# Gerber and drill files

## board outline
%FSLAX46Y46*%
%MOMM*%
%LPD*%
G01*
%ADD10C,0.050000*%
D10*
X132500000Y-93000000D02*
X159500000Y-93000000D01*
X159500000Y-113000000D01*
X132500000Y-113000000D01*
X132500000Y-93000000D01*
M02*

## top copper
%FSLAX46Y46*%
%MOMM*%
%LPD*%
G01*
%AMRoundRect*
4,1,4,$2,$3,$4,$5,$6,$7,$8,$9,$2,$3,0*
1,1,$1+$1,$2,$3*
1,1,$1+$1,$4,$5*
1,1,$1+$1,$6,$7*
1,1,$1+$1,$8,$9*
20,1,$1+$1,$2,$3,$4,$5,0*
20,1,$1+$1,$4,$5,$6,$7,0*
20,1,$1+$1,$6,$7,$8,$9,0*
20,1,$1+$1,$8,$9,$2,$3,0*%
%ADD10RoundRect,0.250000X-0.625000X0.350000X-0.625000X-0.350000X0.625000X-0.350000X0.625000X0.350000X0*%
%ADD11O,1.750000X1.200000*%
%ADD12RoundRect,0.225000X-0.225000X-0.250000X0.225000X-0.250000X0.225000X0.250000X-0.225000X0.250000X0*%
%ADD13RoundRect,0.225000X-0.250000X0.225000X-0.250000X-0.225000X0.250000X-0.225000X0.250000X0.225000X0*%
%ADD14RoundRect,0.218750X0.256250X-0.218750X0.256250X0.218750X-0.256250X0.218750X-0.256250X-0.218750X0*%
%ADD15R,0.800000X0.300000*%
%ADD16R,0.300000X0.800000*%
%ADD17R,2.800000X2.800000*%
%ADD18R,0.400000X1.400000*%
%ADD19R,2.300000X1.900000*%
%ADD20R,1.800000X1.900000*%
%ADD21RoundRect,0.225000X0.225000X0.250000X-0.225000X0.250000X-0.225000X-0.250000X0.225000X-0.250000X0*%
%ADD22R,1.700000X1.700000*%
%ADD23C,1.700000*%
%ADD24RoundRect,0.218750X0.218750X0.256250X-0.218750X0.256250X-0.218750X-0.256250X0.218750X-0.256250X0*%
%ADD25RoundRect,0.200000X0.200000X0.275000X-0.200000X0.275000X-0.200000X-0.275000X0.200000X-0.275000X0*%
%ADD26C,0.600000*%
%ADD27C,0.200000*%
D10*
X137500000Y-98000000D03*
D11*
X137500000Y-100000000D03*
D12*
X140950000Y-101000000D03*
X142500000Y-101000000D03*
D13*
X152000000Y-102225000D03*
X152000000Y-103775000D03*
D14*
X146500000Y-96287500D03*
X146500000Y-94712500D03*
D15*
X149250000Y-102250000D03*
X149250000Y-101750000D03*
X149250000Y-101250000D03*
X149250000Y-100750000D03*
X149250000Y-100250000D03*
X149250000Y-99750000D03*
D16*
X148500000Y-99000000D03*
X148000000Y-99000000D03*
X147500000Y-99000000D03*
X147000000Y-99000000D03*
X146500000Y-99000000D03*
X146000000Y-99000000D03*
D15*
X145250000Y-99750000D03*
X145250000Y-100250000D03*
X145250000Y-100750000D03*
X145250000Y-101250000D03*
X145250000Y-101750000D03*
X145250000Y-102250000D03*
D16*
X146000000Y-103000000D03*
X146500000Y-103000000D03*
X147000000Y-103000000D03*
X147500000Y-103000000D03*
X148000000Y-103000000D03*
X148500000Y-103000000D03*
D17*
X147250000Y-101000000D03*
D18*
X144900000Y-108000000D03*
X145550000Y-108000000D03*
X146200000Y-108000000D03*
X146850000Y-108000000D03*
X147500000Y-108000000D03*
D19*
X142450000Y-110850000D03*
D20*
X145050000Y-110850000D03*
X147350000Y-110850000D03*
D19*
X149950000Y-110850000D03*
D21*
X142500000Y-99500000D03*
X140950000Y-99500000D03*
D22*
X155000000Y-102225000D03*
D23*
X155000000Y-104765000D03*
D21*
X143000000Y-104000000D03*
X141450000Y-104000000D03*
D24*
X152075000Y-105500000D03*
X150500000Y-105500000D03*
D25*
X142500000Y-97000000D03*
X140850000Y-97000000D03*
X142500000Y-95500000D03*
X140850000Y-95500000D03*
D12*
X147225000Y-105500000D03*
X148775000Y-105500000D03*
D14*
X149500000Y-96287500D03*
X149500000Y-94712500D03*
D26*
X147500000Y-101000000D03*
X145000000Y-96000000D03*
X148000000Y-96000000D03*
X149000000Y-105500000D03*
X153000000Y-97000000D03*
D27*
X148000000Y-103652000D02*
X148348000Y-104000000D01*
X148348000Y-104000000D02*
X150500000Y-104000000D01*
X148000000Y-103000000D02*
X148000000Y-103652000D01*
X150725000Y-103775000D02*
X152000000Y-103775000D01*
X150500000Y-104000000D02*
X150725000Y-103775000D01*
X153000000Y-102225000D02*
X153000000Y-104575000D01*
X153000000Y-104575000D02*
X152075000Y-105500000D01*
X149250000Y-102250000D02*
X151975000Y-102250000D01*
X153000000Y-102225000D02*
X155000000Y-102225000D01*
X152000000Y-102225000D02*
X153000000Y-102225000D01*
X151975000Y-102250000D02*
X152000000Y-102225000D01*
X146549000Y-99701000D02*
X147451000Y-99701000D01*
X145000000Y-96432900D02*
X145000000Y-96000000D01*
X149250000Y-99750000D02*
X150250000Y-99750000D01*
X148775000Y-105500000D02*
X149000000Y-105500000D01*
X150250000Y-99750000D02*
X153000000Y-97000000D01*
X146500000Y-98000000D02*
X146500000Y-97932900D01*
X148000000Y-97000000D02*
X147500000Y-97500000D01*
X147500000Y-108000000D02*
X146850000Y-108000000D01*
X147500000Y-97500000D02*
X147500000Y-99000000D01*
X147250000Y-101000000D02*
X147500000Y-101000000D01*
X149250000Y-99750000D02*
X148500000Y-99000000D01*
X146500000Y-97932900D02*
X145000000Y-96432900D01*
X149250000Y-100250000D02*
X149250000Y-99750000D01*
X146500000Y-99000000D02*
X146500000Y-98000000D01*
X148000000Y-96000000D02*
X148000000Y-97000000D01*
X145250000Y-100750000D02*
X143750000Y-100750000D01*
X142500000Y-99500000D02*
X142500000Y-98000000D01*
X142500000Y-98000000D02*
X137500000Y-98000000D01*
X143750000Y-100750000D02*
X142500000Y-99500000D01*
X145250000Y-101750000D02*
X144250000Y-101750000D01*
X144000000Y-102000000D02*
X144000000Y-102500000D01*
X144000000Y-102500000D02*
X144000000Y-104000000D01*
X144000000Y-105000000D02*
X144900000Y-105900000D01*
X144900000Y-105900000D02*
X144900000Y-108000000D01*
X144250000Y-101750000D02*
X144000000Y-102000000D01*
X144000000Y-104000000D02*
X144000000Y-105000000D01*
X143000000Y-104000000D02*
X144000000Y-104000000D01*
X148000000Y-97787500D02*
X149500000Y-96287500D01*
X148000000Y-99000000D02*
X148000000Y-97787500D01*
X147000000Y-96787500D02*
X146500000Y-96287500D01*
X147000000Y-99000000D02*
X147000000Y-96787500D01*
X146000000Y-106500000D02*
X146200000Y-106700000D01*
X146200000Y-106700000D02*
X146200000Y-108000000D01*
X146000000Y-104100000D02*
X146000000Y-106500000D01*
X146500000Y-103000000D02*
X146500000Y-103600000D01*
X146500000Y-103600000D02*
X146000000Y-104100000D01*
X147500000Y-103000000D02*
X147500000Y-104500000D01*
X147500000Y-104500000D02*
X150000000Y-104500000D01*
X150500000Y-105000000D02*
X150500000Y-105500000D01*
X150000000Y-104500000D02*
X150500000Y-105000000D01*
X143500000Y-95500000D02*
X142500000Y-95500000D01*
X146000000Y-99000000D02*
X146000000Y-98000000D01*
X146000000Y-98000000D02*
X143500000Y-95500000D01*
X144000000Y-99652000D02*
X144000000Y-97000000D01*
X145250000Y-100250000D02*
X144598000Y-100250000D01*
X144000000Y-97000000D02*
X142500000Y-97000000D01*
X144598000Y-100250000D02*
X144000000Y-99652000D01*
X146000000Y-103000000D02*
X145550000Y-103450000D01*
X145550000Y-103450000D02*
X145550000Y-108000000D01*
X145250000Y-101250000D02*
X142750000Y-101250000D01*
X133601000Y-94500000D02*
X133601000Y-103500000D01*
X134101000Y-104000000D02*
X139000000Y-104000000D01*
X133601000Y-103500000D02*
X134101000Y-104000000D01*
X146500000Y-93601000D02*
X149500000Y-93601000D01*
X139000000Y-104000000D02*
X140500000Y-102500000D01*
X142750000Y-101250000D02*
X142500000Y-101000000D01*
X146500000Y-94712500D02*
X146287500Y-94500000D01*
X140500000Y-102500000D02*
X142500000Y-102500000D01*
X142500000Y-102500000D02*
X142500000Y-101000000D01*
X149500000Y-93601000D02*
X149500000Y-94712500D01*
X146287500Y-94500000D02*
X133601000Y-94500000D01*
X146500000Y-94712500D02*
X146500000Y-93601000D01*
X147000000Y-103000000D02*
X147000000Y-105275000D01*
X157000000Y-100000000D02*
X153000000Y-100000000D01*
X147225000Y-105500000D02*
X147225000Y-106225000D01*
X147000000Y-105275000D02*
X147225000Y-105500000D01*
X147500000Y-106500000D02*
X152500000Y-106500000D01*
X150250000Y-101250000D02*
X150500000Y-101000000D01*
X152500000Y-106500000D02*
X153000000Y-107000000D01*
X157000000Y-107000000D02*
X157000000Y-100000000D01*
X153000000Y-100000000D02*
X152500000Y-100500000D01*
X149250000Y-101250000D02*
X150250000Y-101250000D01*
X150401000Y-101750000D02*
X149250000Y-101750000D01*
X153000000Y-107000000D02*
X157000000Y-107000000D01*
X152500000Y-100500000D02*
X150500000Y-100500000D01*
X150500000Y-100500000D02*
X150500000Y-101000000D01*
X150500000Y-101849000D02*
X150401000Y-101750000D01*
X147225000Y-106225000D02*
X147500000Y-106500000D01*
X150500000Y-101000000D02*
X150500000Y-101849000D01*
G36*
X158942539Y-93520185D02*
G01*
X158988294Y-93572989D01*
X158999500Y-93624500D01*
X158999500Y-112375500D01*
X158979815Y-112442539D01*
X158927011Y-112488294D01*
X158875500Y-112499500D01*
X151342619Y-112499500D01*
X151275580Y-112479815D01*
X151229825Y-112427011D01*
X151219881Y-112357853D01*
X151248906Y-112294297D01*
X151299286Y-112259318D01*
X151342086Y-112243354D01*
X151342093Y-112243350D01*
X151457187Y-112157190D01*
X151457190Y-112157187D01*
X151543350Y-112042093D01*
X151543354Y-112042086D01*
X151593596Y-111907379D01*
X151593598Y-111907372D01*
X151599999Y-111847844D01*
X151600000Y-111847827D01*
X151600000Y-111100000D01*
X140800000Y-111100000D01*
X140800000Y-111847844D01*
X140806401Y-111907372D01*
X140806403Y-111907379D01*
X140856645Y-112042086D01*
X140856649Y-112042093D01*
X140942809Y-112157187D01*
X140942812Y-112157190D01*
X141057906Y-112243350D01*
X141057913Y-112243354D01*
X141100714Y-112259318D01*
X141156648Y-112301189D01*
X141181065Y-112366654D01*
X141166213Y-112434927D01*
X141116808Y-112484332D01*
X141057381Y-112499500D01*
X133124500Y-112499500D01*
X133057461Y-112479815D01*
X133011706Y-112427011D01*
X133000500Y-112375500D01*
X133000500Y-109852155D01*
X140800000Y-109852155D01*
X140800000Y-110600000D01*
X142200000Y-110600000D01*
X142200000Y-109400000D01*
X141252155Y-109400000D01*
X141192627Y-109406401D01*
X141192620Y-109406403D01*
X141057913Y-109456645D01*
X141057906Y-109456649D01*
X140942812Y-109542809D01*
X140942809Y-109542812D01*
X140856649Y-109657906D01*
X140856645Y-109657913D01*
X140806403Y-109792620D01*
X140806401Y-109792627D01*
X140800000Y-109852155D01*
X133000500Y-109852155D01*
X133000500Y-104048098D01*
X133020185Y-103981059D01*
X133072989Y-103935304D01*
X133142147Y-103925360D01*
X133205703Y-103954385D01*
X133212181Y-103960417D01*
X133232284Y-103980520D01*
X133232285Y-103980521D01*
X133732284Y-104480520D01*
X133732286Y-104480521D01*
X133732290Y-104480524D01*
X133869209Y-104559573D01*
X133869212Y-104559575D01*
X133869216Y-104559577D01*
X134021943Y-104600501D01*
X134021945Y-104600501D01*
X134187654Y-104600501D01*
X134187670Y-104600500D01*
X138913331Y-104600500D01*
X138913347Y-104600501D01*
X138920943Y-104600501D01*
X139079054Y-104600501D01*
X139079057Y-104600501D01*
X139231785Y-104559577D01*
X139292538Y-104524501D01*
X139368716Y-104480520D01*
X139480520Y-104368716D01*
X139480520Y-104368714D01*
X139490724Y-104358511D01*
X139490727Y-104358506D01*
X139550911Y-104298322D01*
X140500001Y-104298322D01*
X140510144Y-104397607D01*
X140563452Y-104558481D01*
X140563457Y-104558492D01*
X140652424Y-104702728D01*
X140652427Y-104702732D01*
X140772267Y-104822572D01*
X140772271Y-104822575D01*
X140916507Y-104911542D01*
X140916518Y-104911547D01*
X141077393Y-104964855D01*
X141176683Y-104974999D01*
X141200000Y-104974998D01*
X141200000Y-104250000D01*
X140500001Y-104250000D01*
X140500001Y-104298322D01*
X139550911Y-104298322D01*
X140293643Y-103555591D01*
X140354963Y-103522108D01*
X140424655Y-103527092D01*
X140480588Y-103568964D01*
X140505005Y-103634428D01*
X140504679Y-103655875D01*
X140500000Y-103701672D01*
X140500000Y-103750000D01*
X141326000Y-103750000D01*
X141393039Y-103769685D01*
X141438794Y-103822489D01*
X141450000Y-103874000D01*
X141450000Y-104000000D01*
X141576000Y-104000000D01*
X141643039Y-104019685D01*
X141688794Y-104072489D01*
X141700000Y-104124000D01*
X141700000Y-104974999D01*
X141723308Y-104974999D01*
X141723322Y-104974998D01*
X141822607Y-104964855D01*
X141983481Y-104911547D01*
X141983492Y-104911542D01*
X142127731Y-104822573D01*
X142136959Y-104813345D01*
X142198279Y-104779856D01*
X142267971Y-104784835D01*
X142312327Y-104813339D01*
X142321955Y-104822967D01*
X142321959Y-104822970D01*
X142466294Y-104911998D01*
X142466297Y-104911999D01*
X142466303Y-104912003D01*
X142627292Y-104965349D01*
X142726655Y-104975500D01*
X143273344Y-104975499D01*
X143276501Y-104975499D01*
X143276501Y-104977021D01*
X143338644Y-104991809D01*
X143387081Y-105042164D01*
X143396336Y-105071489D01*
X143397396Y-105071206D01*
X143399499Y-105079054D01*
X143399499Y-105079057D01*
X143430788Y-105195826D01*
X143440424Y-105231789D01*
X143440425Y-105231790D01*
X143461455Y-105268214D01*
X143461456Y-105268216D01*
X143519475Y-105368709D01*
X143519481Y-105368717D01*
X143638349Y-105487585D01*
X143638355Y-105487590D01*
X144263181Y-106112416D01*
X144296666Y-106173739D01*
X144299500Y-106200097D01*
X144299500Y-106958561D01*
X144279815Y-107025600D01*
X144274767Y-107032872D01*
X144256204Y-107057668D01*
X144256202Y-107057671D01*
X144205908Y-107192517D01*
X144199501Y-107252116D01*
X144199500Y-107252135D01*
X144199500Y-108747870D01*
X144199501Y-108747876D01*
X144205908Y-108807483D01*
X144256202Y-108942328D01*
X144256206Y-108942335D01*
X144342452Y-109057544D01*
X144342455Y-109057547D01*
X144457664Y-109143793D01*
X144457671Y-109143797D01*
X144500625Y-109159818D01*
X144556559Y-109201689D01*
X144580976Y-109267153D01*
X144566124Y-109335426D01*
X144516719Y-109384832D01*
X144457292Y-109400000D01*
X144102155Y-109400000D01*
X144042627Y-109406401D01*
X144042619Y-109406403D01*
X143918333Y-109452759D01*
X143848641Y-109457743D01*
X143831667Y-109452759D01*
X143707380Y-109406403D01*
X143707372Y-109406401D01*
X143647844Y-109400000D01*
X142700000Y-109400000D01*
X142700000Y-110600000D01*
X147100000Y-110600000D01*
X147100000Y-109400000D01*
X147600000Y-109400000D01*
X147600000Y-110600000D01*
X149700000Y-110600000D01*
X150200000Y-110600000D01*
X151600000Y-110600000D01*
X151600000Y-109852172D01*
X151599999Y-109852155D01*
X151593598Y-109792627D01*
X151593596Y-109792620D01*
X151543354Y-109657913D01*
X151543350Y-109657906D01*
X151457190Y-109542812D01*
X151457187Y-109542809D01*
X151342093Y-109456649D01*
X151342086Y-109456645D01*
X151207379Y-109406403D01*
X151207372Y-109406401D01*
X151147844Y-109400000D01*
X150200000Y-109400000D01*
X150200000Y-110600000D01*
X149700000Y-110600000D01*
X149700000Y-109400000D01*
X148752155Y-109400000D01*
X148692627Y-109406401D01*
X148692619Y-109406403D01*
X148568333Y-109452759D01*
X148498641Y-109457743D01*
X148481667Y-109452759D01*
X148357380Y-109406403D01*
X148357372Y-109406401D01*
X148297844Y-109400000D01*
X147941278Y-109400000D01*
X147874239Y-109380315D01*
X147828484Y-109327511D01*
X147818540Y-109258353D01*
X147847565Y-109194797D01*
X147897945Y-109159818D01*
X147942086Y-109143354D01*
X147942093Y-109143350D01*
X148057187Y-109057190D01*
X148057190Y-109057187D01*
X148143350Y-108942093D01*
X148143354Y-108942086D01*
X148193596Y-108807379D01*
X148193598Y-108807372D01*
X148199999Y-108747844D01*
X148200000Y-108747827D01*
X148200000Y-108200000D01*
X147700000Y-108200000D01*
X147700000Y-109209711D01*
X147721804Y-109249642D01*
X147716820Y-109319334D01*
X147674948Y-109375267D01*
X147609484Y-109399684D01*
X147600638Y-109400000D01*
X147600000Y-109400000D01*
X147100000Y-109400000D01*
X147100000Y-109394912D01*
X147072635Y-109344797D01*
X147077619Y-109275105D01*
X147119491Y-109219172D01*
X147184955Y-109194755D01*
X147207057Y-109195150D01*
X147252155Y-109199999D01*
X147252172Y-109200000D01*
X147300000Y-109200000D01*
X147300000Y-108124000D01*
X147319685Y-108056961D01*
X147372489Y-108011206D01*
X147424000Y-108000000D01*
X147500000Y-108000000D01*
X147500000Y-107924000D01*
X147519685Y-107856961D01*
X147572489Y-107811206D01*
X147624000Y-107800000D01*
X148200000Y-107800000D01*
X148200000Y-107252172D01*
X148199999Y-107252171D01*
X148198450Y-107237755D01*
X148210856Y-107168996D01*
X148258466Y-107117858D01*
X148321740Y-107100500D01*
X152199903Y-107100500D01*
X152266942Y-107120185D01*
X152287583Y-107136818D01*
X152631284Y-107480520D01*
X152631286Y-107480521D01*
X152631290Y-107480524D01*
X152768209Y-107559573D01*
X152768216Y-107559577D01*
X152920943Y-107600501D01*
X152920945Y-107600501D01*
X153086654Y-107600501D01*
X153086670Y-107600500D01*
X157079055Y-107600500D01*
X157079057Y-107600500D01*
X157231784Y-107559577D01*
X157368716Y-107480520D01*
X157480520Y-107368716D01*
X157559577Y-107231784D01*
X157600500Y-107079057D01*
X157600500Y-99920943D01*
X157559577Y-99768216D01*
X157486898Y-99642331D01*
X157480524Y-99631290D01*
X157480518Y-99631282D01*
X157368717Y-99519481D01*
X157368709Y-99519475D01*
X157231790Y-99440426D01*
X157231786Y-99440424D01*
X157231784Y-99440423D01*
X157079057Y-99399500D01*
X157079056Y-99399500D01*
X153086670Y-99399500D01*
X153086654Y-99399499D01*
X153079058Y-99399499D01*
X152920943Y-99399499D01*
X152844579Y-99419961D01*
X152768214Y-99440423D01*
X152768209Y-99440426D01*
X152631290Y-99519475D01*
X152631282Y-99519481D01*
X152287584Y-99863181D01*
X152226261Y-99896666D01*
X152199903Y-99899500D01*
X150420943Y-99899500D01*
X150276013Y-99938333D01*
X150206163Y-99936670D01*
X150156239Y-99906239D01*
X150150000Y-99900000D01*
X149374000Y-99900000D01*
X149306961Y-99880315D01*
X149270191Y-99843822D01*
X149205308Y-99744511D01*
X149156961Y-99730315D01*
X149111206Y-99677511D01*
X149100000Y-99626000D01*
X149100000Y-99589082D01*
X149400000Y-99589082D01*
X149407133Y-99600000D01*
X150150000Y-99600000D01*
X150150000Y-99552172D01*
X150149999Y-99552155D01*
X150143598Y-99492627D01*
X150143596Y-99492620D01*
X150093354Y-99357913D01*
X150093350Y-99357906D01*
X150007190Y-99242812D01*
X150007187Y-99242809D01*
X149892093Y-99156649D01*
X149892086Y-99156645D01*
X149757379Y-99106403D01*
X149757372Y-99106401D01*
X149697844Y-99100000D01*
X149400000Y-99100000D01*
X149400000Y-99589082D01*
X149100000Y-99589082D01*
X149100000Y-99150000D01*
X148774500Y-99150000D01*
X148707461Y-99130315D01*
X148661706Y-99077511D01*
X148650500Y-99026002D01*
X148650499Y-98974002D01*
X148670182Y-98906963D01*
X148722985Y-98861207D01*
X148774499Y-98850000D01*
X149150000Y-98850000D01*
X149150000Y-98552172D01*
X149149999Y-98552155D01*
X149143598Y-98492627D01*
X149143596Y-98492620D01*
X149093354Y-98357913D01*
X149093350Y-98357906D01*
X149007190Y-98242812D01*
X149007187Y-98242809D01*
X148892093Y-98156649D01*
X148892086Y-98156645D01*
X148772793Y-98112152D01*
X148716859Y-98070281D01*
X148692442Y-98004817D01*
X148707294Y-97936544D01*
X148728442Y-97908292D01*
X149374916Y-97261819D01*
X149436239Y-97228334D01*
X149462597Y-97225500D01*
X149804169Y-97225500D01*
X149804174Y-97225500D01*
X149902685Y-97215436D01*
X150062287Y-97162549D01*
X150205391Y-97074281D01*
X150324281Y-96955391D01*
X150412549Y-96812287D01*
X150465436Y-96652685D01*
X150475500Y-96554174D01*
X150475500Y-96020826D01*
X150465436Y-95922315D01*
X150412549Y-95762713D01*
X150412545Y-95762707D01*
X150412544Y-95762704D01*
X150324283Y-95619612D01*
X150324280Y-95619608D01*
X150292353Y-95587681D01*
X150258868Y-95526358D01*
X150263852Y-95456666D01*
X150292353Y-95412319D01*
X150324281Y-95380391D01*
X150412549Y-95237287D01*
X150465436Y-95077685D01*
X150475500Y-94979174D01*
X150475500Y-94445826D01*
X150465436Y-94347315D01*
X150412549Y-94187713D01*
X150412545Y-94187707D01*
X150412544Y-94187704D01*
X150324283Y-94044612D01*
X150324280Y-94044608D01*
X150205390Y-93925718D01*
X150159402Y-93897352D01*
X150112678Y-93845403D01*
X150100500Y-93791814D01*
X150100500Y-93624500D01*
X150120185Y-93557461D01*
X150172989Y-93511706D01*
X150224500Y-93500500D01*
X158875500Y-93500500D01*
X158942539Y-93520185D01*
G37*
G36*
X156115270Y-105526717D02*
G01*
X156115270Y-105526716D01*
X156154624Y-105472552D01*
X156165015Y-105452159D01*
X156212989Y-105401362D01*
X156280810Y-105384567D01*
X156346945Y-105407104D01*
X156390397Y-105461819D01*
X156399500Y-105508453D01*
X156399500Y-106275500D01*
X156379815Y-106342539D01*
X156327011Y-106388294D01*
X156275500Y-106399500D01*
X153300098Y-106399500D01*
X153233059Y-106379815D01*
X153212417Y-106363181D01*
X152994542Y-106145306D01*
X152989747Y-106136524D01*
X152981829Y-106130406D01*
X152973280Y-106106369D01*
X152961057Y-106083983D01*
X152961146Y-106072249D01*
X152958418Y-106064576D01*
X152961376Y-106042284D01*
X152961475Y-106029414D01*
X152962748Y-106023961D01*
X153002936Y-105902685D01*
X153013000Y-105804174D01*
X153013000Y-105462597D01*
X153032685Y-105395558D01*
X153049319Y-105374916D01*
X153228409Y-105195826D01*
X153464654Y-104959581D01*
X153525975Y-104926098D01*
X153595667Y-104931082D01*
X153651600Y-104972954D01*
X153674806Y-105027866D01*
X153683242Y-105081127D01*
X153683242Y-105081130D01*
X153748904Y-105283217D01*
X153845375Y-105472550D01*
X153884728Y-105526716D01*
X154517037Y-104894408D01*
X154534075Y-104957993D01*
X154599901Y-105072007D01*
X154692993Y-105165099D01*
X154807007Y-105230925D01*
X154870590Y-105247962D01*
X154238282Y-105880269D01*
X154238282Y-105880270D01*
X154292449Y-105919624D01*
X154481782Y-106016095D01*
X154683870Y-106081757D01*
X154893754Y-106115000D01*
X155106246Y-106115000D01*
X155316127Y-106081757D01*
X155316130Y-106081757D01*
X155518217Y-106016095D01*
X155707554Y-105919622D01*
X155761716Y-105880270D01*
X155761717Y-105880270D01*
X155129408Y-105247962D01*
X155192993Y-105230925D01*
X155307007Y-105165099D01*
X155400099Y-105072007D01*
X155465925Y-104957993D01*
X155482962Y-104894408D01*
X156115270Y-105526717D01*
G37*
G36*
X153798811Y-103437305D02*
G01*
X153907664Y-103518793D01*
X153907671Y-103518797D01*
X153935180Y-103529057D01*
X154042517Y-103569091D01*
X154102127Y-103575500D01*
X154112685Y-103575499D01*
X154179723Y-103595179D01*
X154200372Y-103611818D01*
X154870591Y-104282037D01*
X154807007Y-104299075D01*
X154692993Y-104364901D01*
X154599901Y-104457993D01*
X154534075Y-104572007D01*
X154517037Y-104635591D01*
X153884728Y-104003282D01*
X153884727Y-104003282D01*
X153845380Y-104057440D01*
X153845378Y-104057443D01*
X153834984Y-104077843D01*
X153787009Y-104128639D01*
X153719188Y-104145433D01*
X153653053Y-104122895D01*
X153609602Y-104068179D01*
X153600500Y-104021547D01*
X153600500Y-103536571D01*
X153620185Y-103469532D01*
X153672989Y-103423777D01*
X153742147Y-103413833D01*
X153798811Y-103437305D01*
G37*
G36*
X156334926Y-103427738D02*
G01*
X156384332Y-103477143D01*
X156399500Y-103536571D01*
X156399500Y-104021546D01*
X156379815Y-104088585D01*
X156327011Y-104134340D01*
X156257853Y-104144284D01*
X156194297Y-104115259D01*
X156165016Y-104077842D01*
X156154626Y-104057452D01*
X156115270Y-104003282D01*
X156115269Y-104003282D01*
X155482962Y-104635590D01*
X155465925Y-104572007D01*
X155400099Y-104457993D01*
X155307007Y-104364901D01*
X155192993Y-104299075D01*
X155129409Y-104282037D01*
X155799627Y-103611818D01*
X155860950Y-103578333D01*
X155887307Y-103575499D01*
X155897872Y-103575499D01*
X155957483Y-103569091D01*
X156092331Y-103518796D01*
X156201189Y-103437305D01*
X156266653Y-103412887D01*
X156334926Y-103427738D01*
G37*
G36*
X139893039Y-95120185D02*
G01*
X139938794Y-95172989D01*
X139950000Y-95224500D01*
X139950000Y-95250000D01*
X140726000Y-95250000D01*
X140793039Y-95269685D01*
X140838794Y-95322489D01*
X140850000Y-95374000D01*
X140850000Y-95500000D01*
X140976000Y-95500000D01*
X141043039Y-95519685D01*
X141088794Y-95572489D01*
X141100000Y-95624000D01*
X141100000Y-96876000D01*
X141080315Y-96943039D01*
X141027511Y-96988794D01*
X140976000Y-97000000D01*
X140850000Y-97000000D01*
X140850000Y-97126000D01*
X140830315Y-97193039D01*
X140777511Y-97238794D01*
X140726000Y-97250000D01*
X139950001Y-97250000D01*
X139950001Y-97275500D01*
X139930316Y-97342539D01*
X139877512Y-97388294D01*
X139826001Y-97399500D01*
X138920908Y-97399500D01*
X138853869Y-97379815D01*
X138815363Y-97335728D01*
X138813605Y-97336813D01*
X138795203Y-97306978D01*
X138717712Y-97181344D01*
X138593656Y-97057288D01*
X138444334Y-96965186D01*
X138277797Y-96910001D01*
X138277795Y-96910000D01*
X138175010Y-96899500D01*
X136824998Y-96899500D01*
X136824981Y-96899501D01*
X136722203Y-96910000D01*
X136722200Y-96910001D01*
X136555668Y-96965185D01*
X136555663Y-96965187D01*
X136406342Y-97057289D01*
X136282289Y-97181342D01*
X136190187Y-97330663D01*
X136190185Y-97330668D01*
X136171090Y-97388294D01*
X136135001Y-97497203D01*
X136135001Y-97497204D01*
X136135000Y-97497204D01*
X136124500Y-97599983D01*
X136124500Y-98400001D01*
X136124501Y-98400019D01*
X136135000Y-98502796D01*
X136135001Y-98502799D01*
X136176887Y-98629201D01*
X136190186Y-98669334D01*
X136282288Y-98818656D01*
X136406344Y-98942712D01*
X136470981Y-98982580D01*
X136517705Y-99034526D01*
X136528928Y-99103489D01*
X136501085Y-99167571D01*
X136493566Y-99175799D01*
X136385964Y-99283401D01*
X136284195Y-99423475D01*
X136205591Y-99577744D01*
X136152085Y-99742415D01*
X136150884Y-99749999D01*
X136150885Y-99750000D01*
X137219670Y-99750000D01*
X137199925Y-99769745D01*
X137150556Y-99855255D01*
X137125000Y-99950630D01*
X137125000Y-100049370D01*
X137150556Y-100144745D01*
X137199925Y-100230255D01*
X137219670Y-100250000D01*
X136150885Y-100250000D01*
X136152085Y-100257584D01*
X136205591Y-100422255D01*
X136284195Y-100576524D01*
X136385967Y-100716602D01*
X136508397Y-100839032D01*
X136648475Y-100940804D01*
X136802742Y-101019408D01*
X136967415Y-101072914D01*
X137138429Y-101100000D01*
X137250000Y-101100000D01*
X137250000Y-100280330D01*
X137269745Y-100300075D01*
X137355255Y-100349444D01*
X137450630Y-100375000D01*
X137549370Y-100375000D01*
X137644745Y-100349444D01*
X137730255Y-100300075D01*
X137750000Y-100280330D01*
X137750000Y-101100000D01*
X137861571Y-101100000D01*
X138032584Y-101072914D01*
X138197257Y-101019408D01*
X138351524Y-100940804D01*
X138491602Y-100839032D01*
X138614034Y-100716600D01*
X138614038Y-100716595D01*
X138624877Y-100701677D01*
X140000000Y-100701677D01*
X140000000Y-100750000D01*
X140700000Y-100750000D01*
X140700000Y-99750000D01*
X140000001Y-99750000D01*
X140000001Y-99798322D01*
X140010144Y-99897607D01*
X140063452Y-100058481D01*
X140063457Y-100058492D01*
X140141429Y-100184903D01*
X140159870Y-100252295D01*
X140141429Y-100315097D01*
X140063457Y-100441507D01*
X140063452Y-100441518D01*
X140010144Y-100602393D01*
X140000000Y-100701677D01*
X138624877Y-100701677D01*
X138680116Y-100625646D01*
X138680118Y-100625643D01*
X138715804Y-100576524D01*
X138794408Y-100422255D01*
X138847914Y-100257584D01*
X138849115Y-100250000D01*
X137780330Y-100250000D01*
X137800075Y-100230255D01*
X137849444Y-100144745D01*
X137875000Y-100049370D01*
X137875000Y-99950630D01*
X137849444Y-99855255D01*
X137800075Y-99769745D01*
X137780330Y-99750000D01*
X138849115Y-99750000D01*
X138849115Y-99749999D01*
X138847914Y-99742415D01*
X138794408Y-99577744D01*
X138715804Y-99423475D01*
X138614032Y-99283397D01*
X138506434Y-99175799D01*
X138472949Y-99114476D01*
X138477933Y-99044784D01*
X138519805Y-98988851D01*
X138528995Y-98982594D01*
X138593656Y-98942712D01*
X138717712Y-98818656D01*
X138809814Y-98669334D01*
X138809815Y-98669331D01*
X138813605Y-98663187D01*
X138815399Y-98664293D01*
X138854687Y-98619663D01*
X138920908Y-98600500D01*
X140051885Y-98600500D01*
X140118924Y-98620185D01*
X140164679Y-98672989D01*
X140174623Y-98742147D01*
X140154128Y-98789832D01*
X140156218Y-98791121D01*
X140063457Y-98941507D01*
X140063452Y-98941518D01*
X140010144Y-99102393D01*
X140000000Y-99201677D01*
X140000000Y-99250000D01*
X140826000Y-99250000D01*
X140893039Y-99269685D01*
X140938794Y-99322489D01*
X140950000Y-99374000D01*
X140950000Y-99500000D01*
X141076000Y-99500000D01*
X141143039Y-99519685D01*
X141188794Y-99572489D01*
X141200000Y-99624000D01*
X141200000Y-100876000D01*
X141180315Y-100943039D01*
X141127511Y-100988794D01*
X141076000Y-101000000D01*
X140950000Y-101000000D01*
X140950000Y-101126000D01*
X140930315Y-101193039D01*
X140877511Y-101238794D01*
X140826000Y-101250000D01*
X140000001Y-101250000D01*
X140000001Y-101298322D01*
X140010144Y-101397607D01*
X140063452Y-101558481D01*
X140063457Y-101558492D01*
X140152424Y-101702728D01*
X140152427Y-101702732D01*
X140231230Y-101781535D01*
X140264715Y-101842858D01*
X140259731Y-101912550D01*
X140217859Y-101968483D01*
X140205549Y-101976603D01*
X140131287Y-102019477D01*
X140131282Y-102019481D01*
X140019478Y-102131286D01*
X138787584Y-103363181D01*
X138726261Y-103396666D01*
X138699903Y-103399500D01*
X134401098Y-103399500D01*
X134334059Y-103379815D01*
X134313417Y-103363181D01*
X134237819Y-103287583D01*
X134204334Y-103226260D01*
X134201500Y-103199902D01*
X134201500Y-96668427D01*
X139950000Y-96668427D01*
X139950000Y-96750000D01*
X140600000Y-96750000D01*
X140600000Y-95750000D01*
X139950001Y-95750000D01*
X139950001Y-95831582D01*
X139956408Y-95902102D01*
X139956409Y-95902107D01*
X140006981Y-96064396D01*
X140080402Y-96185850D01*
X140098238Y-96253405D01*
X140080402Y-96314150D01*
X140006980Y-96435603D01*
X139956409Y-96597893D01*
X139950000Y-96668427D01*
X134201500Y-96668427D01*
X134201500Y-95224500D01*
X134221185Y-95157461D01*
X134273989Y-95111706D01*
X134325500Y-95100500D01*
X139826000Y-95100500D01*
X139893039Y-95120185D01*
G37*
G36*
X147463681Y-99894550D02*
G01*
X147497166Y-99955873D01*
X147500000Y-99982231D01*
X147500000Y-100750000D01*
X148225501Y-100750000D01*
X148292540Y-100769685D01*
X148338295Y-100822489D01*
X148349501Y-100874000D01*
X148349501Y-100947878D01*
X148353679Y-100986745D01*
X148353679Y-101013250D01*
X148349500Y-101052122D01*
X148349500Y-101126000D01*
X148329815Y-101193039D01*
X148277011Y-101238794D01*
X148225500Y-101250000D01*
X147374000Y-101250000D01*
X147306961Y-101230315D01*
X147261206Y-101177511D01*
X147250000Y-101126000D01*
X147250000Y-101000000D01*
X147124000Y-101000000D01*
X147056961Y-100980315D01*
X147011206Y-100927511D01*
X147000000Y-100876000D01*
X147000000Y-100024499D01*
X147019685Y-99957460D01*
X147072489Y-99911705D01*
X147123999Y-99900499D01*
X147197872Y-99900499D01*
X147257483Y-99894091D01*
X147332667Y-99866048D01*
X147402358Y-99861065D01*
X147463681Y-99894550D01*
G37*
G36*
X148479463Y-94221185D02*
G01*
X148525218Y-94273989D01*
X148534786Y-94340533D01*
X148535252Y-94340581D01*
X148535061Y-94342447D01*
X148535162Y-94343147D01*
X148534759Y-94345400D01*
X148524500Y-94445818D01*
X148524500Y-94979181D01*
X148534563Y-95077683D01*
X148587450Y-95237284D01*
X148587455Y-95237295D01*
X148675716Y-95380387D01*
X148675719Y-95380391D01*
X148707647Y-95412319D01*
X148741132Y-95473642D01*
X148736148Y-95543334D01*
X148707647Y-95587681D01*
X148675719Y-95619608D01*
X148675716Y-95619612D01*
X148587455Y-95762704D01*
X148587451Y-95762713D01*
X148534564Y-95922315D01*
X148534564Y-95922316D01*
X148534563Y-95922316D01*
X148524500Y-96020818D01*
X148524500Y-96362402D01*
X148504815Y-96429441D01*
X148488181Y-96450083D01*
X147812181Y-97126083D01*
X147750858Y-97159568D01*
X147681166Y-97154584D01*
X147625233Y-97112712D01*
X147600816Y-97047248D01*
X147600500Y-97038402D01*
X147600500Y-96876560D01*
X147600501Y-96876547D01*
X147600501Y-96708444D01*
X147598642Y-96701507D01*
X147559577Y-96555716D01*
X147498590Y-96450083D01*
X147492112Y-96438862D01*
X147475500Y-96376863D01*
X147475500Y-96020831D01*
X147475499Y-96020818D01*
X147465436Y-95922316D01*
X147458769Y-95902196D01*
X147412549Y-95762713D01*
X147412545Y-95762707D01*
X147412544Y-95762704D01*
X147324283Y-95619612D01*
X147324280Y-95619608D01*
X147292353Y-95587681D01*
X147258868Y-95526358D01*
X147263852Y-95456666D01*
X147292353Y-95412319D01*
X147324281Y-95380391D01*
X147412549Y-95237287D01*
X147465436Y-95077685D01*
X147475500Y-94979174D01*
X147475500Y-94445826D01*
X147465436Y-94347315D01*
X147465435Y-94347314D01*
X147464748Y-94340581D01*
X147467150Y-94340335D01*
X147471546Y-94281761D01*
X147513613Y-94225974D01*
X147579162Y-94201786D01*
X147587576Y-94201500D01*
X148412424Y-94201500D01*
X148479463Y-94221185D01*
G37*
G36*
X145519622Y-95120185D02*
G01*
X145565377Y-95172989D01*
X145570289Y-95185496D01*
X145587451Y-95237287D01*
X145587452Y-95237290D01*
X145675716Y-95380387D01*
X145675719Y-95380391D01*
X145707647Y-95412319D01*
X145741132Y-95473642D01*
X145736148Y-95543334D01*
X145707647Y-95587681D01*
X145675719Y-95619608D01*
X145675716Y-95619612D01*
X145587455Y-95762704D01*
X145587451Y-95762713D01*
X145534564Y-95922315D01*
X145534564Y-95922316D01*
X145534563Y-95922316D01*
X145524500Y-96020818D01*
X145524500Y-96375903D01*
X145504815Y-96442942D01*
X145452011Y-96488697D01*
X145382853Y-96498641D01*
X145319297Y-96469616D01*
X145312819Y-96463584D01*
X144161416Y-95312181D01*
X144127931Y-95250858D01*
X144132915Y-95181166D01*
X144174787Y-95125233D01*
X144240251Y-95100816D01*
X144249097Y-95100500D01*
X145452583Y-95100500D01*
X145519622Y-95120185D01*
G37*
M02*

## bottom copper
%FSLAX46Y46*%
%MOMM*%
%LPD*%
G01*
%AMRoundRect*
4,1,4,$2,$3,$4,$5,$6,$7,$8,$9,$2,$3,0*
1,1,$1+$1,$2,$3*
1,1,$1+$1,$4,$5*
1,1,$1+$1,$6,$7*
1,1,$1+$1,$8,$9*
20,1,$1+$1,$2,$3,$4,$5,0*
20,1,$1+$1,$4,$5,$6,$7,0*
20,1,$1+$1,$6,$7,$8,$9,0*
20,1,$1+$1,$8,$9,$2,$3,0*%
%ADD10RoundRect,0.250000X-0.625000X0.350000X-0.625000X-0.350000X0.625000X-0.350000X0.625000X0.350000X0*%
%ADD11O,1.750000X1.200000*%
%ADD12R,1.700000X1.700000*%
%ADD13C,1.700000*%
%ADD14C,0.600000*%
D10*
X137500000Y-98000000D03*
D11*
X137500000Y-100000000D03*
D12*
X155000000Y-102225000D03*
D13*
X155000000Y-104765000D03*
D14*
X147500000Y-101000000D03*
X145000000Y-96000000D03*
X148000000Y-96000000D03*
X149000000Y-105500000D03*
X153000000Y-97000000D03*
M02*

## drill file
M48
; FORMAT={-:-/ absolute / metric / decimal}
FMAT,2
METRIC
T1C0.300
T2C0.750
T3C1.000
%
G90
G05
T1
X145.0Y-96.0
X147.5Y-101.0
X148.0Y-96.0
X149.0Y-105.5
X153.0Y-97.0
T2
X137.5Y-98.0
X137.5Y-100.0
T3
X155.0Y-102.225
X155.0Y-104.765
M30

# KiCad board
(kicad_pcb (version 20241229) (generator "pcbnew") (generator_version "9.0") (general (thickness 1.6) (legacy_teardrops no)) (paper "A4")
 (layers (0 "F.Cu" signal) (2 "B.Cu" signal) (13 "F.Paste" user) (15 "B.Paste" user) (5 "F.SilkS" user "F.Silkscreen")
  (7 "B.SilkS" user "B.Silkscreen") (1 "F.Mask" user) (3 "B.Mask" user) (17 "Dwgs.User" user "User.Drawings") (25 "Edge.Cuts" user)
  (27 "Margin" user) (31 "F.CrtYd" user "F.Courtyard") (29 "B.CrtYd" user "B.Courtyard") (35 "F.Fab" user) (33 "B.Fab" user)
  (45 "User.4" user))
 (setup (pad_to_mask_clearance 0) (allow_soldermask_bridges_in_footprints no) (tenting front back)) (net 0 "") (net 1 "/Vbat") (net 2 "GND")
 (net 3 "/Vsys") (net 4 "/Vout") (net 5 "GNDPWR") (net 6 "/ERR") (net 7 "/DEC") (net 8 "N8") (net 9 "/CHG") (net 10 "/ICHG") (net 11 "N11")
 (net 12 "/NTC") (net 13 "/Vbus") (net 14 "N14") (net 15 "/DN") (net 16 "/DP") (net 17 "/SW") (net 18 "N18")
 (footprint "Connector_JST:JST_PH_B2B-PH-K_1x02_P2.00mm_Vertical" (layer "F.Cu") (at 137.5 98 -90)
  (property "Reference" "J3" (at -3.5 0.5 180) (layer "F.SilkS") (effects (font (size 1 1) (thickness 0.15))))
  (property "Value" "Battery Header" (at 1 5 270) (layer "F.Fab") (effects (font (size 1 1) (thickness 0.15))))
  (pad "1" thru_hole roundrect (at 0 0 270) (size 1.2 1.75) (drill 0.75) (layers "*.Cu" "*.Mask") (remove_unused_layers no)
   (roundrect_rratio 0.208333) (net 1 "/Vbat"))
  (pad "2" thru_hole oval (at 2 0 270) (size 1.2 1.75) (drill 0.75) (layers "*.Cu" "*.Mask") (remove_unused_layers no) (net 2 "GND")))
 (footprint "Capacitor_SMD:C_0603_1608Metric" (layer "F.Cu") (at 141.725 101)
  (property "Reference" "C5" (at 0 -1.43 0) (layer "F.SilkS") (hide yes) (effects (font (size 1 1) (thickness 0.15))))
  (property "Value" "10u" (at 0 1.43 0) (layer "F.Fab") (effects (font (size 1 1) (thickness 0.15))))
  (pad "1" smd roundrect (at -0.775 0) (size 0.9 0.95) (layers "F.Cu" "F.Mask" "F.Paste") (roundrect_rratio 0.25) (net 2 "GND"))
  (pad "2" smd roundrect (at 0.775 0) (size 0.9 0.95) (layers "F.Cu" "F.Mask" "F.Paste") (roundrect_rratio 0.25) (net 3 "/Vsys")))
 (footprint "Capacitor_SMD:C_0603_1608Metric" (layer "F.Cu") (at 152 103 -90)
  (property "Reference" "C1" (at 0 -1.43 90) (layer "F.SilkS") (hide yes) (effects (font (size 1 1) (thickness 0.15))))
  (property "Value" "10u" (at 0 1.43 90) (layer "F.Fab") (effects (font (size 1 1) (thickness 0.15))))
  (pad "1" smd roundrect (at -0.775 0 270) (size 0.9 0.95) (layers "F.Cu" "F.Mask" "F.Paste") (roundrect_rratio 0.25) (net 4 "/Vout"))
  (pad "2" smd roundrect (at 0.775 0 270) (size 0.9 0.95) (layers "F.Cu" "F.Mask" "F.Paste") (roundrect_rratio 0.25) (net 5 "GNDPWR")))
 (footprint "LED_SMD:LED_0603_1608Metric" (layer "F.Cu") (at 146.5 95.5 90)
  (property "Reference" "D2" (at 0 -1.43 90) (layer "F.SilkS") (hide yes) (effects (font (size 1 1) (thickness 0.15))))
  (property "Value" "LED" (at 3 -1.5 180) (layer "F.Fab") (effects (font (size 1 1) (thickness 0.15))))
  (pad "1" smd roundrect (at -0.7875 0 90) (size 0.875 0.95) (layers "F.Cu" "F.Mask" "F.Paste") (roundrect_rratio 0.25) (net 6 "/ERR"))
  (pad "2" smd roundrect (at 0.7875 0 90) (size 0.875 0.95) (layers "F.Cu" "F.Mask" "F.Paste") (roundrect_rratio 0.25) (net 3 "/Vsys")))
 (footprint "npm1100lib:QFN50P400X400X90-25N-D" (layer "F.Cu") (at 147.25 101 180)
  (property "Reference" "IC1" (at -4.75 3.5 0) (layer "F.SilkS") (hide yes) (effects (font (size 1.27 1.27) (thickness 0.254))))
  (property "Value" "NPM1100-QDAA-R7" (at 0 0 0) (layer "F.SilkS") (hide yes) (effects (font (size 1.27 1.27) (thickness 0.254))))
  (pad "1" smd rect (at -2 -1.25 270) (size 0.3 0.8) (layers "F.Cu" "F.Mask" "F.Paste") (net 4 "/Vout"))
  (pad "2" smd rect (at -2 -0.75 270) (size 0.3 0.8) (layers "F.Cu" "F.Mask" "F.Paste") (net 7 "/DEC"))
  (pad "3" smd rect (at -2 -0.25 270) (size 0.3 0.8) (layers "F.Cu" "F.Mask" "F.Paste") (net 7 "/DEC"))
  (pad "4" smd rect (at -2 0.25 270) (size 0.3 0.8) (layers "F.Cu" "F.Mask" "F.Paste") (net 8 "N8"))
  (pad "5" smd rect (at -2 0.75 270) (size 0.3 0.8) (layers "F.Cu" "F.Mask" "F.Paste") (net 2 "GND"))
  (pad "6" smd rect (at -2 1.25 270) (size 0.3 0.8) (layers "F.Cu" "F.Mask" "F.Paste") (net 2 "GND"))
  (pad "7" smd rect (at -1.25 2 180) (size 0.3 0.8) (layers "F.Cu" "F.Mask" "F.Paste") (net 2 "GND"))
  (pad "8" smd rect (at -0.75 2 180) (size 0.3 0.8) (layers "F.Cu" "F.Mask" "F.Paste") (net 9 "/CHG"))
  (pad "9" smd rect (at -0.25 2 180) (size 0.3 0.8) (layers "F.Cu" "F.Mask" "F.Paste") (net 2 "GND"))
  (pad "10" smd rect (at 0.25 2 180) (size 0.3 0.8) (layers "F.Cu" "F.Mask" "F.Paste") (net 6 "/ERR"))
  (pad "11" smd rect (at 0.75 2 180) (size 0.3 0.8) (layers "F.Cu" "F.Mask" "F.Paste") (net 2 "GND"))
  (pad "12" smd rect (at 1.25 2 180) (size 0.3 0.8) (layers "F.Cu" "F.Mask" "F.Paste") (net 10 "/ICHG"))
  (pad "13" smd rect (at 2 1.25 270) (size 0.3 0.8) (layers "F.Cu" "F.Mask" "F.Paste") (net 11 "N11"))
  (pad "14" smd rect (at 2 0.75 270) (size 0.3 0.8) (layers "F.Cu" "F.Mask" "F.Paste") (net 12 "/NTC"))
  (pad "15" smd rect (at 2 0.25 270) (size 0.3 0.8) (layers "F.Cu" "F.Mask" "F.Paste") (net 1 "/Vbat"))
  (pad "16" smd rect (at 2 -0.25 270) (size 0.3 0.8) (layers "F.Cu" "F.Mask" "F.Paste") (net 3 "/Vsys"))
  (pad "17" smd rect (at 2 -0.75 270) (size 0.3 0.8) (layers "F.Cu" "F.Mask" "F.Paste") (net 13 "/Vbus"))
  (pad "18" smd rect (at 2 -1.25 270) (size 0.3 0.8) (layers "F.Cu" "F.Mask" "F.Paste") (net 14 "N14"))
  (pad "19" smd rect (at 1.25 -2 180) (size 0.3 0.8) (layers "F.Cu" "F.Mask" "F.Paste") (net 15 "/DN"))
  (pad "20" smd rect (at 0.75 -2 180) (size 0.3 0.8) (layers "F.Cu" "F.Mask" "F.Paste") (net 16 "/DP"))
  (pad "21" smd rect (at 0.25 -2 180) (size 0.3 0.8) (layers "F.Cu" "F.Mask" "F.Paste") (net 7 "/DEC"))
  (pad "22" smd rect (at -0.25 -2 180) (size 0.3 0.8) (layers "F.Cu" "F.Mask" "F.Paste") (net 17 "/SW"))
  (pad "23" smd rect (at -0.75 -2 180) (size 0.3 0.8) (layers "F.Cu" "F.Mask" "F.Paste") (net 5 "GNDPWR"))
  (pad "24" smd rect (at -1.25 -2 180) (size 0.3 0.8) (layers "F.Cu" "F.Mask" "F.Paste") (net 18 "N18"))
  (pad "25" smd rect (at 0 0 180) (size 2.8 2.8) (layers "F.Cu" "F.Mask" "F.Paste") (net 2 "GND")))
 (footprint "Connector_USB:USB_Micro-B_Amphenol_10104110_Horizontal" (layer "F.Cu") (at 146.2 109.55)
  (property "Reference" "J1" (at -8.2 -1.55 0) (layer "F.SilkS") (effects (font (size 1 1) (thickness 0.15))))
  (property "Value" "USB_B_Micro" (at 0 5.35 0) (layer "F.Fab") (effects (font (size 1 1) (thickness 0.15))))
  (pad "1" smd rect (at -1.3 -1.55) (size 0.4 1.4) (layers "F.Cu" "F.Mask" "F.Paste") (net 13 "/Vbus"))
  (pad "2" smd rect (at -0.65 -1.55) (size 0.4 1.4) (layers "F.Cu" "F.Mask" "F.Paste") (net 15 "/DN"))
  (pad "3" smd rect (at 0 -1.55) (size 0.4 1.4) (layers "F.Cu" "F.Mask" "F.Paste") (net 16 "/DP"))
  (pad "4" smd rect (at 0.65 -1.55) (size 0.4 1.4) (layers "F.Cu" "F.Mask" "F.Paste") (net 2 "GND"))
  (pad "5" smd rect (at 1.3 -1.55) (size 0.4 1.4) (layers "F.Cu" "F.Mask" "F.Paste") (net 2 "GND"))
  (pad "6" smd rect (at -3.75 1.3) (size 2.3 1.9) (layers "F.Cu" "F.Mask" "F.Paste") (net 2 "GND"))
  (pad "6" smd rect (at -1.15 1.3) (size 1.8 1.9) (layers "F.Cu" "F.Mask" "F.Paste") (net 2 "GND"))
  (pad "6" smd rect (at 1.15 1.3) (size 1.8 1.9) (layers "F.Cu" "F.Mask" "F.Paste") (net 2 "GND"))
  (pad "6" smd rect (at 3.75 1.3) (size 2.3 1.9) (layers "F.Cu" "F.Mask" "F.Paste") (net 2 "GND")))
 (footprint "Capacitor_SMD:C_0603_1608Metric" (layer "F.Cu") (at 141.725 99.5 180)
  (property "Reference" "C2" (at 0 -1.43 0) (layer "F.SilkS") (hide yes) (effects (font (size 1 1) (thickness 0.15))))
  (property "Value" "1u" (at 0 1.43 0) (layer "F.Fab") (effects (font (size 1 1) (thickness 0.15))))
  (pad "1" smd roundrect (at -0.775 0 180) (size 0.9 0.95) (layers "F.Cu" "F.Mask" "F.Paste") (roundrect_rratio 0.25) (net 1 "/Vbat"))
  (pad "2" smd roundrect (at 0.775 0 180) (size 0.9 0.95) (layers "F.Cu" "F.Mask" "F.Paste") (roundrect_rratio 0.25) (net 2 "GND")))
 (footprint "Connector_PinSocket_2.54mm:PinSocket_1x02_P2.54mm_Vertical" (layer "F.Cu") (at 155 102.225)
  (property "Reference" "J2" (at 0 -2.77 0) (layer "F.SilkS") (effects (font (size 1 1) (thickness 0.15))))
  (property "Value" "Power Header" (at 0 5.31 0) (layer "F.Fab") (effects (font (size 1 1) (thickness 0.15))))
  (pad "1" thru_hole rect (at 0 0) (size 1.7 1.7) (drill 1) (layers "*.Cu" "*.Mask") (remove_unused_layers no) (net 4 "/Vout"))
  (pad "2" thru_hole circle (at 0 2.54) (size 1.7 1.7) (drill 1) (layers "*.Cu" "*.Mask") (remove_unused_layers no) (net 2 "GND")))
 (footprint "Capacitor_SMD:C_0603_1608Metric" (layer "F.Cu") (at 142.225 104 180)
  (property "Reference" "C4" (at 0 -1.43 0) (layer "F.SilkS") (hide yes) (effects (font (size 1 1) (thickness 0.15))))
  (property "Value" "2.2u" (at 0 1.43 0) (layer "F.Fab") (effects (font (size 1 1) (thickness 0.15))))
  (pad "1" smd roundrect (at -0.775 0 180) (size 0.9 0.95) (layers "F.Cu" "F.Mask" "F.Paste") (roundrect_rratio 0.25) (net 13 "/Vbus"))
  (pad "2" smd roundrect (at 0.775 0 180) (size 0.9 0.95) (layers "F.Cu" "F.Mask" "F.Paste") (roundrect_rratio 0.25) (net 2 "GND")))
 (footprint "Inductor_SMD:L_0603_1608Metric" (layer "F.Cu") (at 151.2875 105.5 180)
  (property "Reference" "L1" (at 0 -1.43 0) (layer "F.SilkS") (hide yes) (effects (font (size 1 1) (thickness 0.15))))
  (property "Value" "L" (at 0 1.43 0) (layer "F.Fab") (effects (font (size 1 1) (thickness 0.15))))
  (pad "1" smd roundrect (at -0.7875 0 180) (size 0.875 0.95) (layers "F.Cu" "F.Mask" "F.Paste") (roundrect_rratio 0.25) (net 4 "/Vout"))
  (pad "2" smd roundrect (at 0.7875 0 180) (size 0.875 0.95) (layers "F.Cu" "F.Mask" "F.Paste") (roundrect_rratio 0.25) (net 17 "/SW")))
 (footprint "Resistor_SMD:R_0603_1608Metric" (layer "F.Cu") (at 141.675 97 180)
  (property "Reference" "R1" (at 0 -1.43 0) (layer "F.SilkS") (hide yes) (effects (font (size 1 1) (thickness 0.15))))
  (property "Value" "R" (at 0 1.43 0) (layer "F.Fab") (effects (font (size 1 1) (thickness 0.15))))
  (pad "1" smd roundrect (at -0.825 0 180) (size 0.8 0.95) (layers "F.Cu" "F.Mask" "F.Paste") (roundrect_rratio 0.25) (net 12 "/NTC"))
  (pad "2" smd roundrect (at 0.825 0 180) (size 0.8 0.95) (layers "F.Cu" "F.Mask" "F.Paste") (roundrect_rratio 0.25) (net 2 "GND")))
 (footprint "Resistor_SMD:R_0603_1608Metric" (layer "F.Cu") (at 141.675 95.5 180)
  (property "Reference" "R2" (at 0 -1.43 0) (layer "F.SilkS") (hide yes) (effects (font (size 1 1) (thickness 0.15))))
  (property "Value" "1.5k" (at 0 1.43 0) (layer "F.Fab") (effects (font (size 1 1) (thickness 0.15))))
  (pad "1" smd roundrect (at -0.825 0 180) (size 0.8 0.95) (layers "F.Cu" "F.Mask" "F.Paste") (roundrect_rratio 0.25) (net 10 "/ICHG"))
  (pad "2" smd roundrect (at 0.825 0 180) (size 0.8 0.95) (layers "F.Cu" "F.Mask" "F.Paste") (roundrect_rratio 0.25) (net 2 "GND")))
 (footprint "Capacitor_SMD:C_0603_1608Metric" (layer "F.Cu") (at 148 105.5)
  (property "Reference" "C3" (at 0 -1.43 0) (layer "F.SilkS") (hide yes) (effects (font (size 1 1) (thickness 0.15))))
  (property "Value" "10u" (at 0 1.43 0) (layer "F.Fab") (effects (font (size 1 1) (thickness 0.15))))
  (pad "1" smd roundrect (at -0.775 0) (size 0.9 0.95) (layers "F.Cu" "F.Mask" "F.Paste") (roundrect_rratio 0.25) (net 7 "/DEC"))
  (pad "2" smd roundrect (at 0.775 0) (size 0.9 0.95) (layers "F.Cu" "F.Mask" "F.Paste") (roundrect_rratio 0.25) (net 2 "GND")))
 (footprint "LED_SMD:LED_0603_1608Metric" (layer "F.Cu") (at 149.5 95.5 90)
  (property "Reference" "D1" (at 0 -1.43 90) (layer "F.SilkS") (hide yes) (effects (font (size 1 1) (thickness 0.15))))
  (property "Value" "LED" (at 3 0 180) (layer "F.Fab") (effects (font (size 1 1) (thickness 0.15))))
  (pad "1" smd roundrect (at -0.7875 0 90) (size 0.875 0.95) (layers "F.Cu" "F.Mask" "F.Paste") (roundrect_rratio 0.25) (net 9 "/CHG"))
  (pad "2" smd roundrect (at 0.7875 0 90) (size 0.875 0.95) (layers "F.Cu" "F.Mask" "F.Paste") (roundrect_rratio 0.25) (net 3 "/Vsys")))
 (gr_rect (start 132.5 93) (end 159.5 113) (stroke (width 0.05) (type default)) (fill no) (layer "Edge.Cuts"))
 (segment (start 148 103.652) (end 148.348 104) (width 0.2) (layer "F.Cu") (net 5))
 (segment (start 148.348 104) (end 150.5 104) (width 0.2) (layer "F.Cu") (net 5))
 (segment (start 148 103) (end 148 103.652) (width 0.2) (layer "F.Cu") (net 5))
 (segment (start 150.725 103.775) (end 152 103.775) (width 0.2) (layer "F.Cu") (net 5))
 (segment (start 150.5 104) (end 150.725 103.775) (width 0.2) (layer "F.Cu") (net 5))
 (segment (start 153 102.225) (end 153 104.575) (width 0.2) (layer "F.Cu") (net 4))
 (segment (start 153 104.575) (end 152.075 105.5) (width 0.2) (layer "F.Cu") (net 4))
 (segment (start 149.25 102.25) (end 151.975 102.25) (width 0.2) (layer "F.Cu") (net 4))
 (segment (start 153 102.225) (end 155 102.225) (width 0.2) (layer "F.Cu") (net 4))
 (segment (start 152 102.225) (end 153 102.225) (width 0.2) (layer "F.Cu") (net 4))
 (segment (start 151.975 102.25) (end 152 102.225) (width 0.2) (layer "F.Cu") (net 4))
 (segment (start 146.549 99.701) (end 147.451 99.701) (width 0.2) (layer "F.Cu") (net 2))
 (segment (start 145 96.4329) (end 145 96) (width 0.2) (layer "F.Cu") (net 2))
 (segment (start 149.25 99.75) (end 150.25 99.75) (width 0.2) (layer "F.Cu") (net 2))
 (segment (start 148.775 105.5) (end 149 105.5) (width 0.2) (layer "F.Cu") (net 2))
 (segment (start 150.25 99.75) (end 153 97) (width 0.2) (layer "F.Cu") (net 2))
 (segment (start 146.5 98) (end 146.5 97.9329) (width 0.2) (layer "F.Cu") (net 2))
 (segment (start 148 97) (end 147.5 97.5) (width 0.2) (layer "F.Cu") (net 2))
 (segment (start 147.5 108) (end 146.85 108) (width 0.2) (layer "F.Cu") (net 2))
 (segment (start 147.5 97.5) (end 147.5 99) (width 0.2) (layer "F.Cu") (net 2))
 (segment (start 147.25 101) (end 147.5 101) (width 0.2) (layer "F.Cu") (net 2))
 (segment (start 149.25 99.75) (end 148.5 99) (width 0.2) (layer "F.Cu") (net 2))
 (segment (start 146.5 97.9329) (end 145 96.4329) (width 0.2) (layer "F.Cu") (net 2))
 (segment (start 149.25 100.25) (end 149.25 99.75) (width 0.2) (layer "F.Cu") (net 2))
 (segment (start 146.5 99) (end 146.5 98) (width 0.2) (layer "F.Cu") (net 2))
 (segment (start 148 96) (end 148 97) (width 0.2) (layer "F.Cu") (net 2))
 (via (at 147.5 101) (size 0.6) (drill 0.3) (layers "F.Cu" "B.Cu") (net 2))
 (via (at 145 96) (size 0.6) (drill 0.3) (layers "F.Cu" "B.Cu") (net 2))
 (via (at 148 96) (size 0.6) (drill 0.3) (layers "F.Cu" "B.Cu") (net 2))
 (via (at 149 105.5) (size 0.6) (drill 0.3) (layers "F.Cu" "B.Cu") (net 2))
 (via (at 153 97) (size 0.6) (drill 0.3) (layers "F.Cu" "B.Cu") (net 2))
 (segment (start 145.25 100.75) (end 143.75 100.75) (width 0.2) (layer "F.Cu") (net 1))
 (segment (start 142.5 99.5) (end 142.5 98) (width 0.2) (layer "F.Cu") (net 1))
 (segment (start 142.5 98) (end 137.5 98) (width 0.2) (layer "F.Cu") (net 1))
 (segment (start 143.75 100.75) (end 142.5 99.5) (width 0.2) (layer "F.Cu") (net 1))
 (segment (start 145.25 101.75) (end 144.25 101.75) (width 0.2) (layer "F.Cu") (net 13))
 (segment (start 144 102) (end 144 102.5) (width 0.2) (layer "F.Cu") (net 13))
 (segment (start 144 102.5) (end 144 104) (width 0.2) (layer "F.Cu") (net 13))
 (segment (start 144 105) (end 144.9 105.9) (width 0.2) (layer "F.Cu") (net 13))
 (segment (start 144.9 105.9) (end 144.9 108) (width 0.2) (layer "F.Cu") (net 13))
 (segment (start 144.25 101.75) (end 144 102) (width 0.2) (layer "F.Cu") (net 13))
 (segment (start 144 104) (end 144 105) (width 0.2) (layer "F.Cu") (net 13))
 (segment (start 143 104) (end 144 104) (width 0.2) (layer "F.Cu") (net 13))
 (segment (start 148 97.7875) (end 149.5 96.2875) (width 0.2) (layer "F.Cu") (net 9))
 (segment (start 148 99) (end 148 97.7875) (width 0.2) (layer "F.Cu") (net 9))
 (segment (start 147 96.7875) (end 146.5 96.2875) (width 0.2) (layer "F.Cu") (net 6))
 (segment (start 147 99) (end 147 96.7875) (width 0.2) (layer "F.Cu") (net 6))
 (segment (start 146 106.5) (end 146.2 106.7) (width 0.2) (layer "F.Cu") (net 16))
 (segment (start 146.2 106.7) (end 146.2 108) (width 0.2) (layer "F.Cu") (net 16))
 (segment (start 146 104.1) (end 146 106.5) (width 0.2) (layer "F.Cu") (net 16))
 (segment (start 146.5 103) (end 146.5 103.6) (width 0.2) (layer "F.Cu") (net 16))
 (segment (start 146.5 103.6) (end 146 104.1) (width 0.2) (layer "F.Cu") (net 16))
 (segment (start 147.5 103) (end 147.5 104.5) (width 0.2) (layer "F.Cu") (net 17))
 (segment (start 147.5 104.5) (end 150 104.5) (width 0.2) (layer "F.Cu") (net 17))
 (segment (start 150.5 105) (end 150.5 105.5) (width 0.2) (layer "F.Cu") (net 17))
 (segment (start 150 104.5) (end 150.5 105) (width 0.2) (layer "F.Cu") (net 17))
 (segment (start 143.5 95.5) (end 142.5 95.5) (width 0.2) (layer "F.Cu") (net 10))
 (segment (start 146 99) (end 146 98) (width 0.2) (layer "F.Cu") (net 10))
 (segment (start 146 98) (end 143.5 95.5) (width 0.2) (layer "F.Cu") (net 10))
 (segment (start 144 99.652) (end 144 97) (width 0.2) (layer "F.Cu") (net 12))
 (segment (start 145.25 100.25) (end 144.598 100.25) (width 0.2) (layer "F.Cu") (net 12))
 (segment (start 144 97) (end 142.5 97) (width 0.2) (layer "F.Cu") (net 12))
 (segment (start 144.598 100.25) (end 144 99.652) (width 0.2) (layer "F.Cu") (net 12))
 (segment (start 146 103) (end 145.55 103.45) (width 0.2) (layer "F.Cu") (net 15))
 (segment (start 145.55 103.45) (end 145.55 108) (width 0.2) (layer "F.Cu") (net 15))
 (segment (start 145.25 101.25) (end 142.75 101.25) (width 0.2) (layer "F.Cu") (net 3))
 (segment (start 133.601 94.5) (end 133.601 103.5) (width 0.2) (layer "F.Cu") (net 3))
 (segment (start 134.101 104) (end 139 104) (width 0.2) (layer "F.Cu") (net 3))
 (segment (start 133.601 103.5) (end 134.101 104) (width 0.2) (layer "F.Cu") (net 3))
 (segment (start 146.5 93.601) (end 149.5 93.601) (width 0.2) (layer "F.Cu") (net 3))
 (segment (start 139 104) (end 140.5 102.5) (width 0.2) (layer "F.Cu") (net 3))
 (segment (start 142.75 101.25) (end 142.5 101) (width 0.2) (layer "F.Cu") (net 3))
 (segment (start 146.5 94.7125) (end 146.2875 94.5) (width 0.2) (layer "F.Cu") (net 3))
 (segment (start 140.5 102.5) (end 142.5 102.5) (width 0.2) (layer "F.Cu") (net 3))
 (segment (start 142.5 102.5) (end 142.5 101) (width 0.2) (layer "F.Cu") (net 3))
 (segment (start 149.5 93.601) (end 149.5 94.7125) (width 0.2) (layer "F.Cu") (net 3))
 (segment (start 146.2875 94.5) (end 133.601 94.5) (width 0.2) (layer "F.Cu") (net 3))
 (segment (start 146.5 94.7125) (end 146.5 93.601) (width 0.2) (layer "F.Cu") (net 3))
 (segment (start 147 103) (end 147 105.275) (width 0.2) (layer "F.Cu") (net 7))
 (segment (start 157 100) (end 153 100) (width 0.2) (layer "F.Cu") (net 7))
 (segment (start 147.225 105.5) (end 147.225 106.225) (width 0.2) (layer "F.Cu") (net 7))
 (segment (start 147 105.275) (end 147.225 105.5) (width 0.2) (layer "F.Cu") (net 7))
 (segment (start 147.5 106.5) (end 152.5 106.5) (width 0.2) (layer "F.Cu") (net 7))
 (segment (start 150.25 101.25) (end 150.5 101) (width 0.2) (layer "F.Cu") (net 7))
 (segment (start 152.5 106.5) (end 153 107) (width 0.2) (layer "F.Cu") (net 7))
 (segment (start 157 107) (end 157 100) (width 0.2) (layer "F.Cu") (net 7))
 (segment (start 153 100) (end 152.5 100.5) (width 0.2) (layer "F.Cu") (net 7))
 (segment (start 149.25 101.25) (end 150.25 101.25) (width 0.2) (layer "F.Cu") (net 7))
 (segment (start 150.401 101.75) (end 149.25 101.75) (width 0.2) (layer "F.Cu") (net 7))
 (segment (start 153 107) (end 157 107) (width 0.2) (layer "F.Cu") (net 7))
 (segment (start 152.5 100.5) (end 150.5 100.5) (width 0.2) (layer "F.Cu") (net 7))
 (segment (start 150.5 100.5) (end 150.5 101) (width 0.2) (layer "F.Cu") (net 7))
 (segment (start 150.5 101.849) (end 150.401 101.75) (width 0.2) (layer "F.Cu") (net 7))
 (segment (start 147.225 106.225) (end 147.5 106.5) (width 0.2) (layer "F.Cu") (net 7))
 (segment (start 150.5 101) (end 150.5 101.849) (width 0.2) (layer "F.Cu") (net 7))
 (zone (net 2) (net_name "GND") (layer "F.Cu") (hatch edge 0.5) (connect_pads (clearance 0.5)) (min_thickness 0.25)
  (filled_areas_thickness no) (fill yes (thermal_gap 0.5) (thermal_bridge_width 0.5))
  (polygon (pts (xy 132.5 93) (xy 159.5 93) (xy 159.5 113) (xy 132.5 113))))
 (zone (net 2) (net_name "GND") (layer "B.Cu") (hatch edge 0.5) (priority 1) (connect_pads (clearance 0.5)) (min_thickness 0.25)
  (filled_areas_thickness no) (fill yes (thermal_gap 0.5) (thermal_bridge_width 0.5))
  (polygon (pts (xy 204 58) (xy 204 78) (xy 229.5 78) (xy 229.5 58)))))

